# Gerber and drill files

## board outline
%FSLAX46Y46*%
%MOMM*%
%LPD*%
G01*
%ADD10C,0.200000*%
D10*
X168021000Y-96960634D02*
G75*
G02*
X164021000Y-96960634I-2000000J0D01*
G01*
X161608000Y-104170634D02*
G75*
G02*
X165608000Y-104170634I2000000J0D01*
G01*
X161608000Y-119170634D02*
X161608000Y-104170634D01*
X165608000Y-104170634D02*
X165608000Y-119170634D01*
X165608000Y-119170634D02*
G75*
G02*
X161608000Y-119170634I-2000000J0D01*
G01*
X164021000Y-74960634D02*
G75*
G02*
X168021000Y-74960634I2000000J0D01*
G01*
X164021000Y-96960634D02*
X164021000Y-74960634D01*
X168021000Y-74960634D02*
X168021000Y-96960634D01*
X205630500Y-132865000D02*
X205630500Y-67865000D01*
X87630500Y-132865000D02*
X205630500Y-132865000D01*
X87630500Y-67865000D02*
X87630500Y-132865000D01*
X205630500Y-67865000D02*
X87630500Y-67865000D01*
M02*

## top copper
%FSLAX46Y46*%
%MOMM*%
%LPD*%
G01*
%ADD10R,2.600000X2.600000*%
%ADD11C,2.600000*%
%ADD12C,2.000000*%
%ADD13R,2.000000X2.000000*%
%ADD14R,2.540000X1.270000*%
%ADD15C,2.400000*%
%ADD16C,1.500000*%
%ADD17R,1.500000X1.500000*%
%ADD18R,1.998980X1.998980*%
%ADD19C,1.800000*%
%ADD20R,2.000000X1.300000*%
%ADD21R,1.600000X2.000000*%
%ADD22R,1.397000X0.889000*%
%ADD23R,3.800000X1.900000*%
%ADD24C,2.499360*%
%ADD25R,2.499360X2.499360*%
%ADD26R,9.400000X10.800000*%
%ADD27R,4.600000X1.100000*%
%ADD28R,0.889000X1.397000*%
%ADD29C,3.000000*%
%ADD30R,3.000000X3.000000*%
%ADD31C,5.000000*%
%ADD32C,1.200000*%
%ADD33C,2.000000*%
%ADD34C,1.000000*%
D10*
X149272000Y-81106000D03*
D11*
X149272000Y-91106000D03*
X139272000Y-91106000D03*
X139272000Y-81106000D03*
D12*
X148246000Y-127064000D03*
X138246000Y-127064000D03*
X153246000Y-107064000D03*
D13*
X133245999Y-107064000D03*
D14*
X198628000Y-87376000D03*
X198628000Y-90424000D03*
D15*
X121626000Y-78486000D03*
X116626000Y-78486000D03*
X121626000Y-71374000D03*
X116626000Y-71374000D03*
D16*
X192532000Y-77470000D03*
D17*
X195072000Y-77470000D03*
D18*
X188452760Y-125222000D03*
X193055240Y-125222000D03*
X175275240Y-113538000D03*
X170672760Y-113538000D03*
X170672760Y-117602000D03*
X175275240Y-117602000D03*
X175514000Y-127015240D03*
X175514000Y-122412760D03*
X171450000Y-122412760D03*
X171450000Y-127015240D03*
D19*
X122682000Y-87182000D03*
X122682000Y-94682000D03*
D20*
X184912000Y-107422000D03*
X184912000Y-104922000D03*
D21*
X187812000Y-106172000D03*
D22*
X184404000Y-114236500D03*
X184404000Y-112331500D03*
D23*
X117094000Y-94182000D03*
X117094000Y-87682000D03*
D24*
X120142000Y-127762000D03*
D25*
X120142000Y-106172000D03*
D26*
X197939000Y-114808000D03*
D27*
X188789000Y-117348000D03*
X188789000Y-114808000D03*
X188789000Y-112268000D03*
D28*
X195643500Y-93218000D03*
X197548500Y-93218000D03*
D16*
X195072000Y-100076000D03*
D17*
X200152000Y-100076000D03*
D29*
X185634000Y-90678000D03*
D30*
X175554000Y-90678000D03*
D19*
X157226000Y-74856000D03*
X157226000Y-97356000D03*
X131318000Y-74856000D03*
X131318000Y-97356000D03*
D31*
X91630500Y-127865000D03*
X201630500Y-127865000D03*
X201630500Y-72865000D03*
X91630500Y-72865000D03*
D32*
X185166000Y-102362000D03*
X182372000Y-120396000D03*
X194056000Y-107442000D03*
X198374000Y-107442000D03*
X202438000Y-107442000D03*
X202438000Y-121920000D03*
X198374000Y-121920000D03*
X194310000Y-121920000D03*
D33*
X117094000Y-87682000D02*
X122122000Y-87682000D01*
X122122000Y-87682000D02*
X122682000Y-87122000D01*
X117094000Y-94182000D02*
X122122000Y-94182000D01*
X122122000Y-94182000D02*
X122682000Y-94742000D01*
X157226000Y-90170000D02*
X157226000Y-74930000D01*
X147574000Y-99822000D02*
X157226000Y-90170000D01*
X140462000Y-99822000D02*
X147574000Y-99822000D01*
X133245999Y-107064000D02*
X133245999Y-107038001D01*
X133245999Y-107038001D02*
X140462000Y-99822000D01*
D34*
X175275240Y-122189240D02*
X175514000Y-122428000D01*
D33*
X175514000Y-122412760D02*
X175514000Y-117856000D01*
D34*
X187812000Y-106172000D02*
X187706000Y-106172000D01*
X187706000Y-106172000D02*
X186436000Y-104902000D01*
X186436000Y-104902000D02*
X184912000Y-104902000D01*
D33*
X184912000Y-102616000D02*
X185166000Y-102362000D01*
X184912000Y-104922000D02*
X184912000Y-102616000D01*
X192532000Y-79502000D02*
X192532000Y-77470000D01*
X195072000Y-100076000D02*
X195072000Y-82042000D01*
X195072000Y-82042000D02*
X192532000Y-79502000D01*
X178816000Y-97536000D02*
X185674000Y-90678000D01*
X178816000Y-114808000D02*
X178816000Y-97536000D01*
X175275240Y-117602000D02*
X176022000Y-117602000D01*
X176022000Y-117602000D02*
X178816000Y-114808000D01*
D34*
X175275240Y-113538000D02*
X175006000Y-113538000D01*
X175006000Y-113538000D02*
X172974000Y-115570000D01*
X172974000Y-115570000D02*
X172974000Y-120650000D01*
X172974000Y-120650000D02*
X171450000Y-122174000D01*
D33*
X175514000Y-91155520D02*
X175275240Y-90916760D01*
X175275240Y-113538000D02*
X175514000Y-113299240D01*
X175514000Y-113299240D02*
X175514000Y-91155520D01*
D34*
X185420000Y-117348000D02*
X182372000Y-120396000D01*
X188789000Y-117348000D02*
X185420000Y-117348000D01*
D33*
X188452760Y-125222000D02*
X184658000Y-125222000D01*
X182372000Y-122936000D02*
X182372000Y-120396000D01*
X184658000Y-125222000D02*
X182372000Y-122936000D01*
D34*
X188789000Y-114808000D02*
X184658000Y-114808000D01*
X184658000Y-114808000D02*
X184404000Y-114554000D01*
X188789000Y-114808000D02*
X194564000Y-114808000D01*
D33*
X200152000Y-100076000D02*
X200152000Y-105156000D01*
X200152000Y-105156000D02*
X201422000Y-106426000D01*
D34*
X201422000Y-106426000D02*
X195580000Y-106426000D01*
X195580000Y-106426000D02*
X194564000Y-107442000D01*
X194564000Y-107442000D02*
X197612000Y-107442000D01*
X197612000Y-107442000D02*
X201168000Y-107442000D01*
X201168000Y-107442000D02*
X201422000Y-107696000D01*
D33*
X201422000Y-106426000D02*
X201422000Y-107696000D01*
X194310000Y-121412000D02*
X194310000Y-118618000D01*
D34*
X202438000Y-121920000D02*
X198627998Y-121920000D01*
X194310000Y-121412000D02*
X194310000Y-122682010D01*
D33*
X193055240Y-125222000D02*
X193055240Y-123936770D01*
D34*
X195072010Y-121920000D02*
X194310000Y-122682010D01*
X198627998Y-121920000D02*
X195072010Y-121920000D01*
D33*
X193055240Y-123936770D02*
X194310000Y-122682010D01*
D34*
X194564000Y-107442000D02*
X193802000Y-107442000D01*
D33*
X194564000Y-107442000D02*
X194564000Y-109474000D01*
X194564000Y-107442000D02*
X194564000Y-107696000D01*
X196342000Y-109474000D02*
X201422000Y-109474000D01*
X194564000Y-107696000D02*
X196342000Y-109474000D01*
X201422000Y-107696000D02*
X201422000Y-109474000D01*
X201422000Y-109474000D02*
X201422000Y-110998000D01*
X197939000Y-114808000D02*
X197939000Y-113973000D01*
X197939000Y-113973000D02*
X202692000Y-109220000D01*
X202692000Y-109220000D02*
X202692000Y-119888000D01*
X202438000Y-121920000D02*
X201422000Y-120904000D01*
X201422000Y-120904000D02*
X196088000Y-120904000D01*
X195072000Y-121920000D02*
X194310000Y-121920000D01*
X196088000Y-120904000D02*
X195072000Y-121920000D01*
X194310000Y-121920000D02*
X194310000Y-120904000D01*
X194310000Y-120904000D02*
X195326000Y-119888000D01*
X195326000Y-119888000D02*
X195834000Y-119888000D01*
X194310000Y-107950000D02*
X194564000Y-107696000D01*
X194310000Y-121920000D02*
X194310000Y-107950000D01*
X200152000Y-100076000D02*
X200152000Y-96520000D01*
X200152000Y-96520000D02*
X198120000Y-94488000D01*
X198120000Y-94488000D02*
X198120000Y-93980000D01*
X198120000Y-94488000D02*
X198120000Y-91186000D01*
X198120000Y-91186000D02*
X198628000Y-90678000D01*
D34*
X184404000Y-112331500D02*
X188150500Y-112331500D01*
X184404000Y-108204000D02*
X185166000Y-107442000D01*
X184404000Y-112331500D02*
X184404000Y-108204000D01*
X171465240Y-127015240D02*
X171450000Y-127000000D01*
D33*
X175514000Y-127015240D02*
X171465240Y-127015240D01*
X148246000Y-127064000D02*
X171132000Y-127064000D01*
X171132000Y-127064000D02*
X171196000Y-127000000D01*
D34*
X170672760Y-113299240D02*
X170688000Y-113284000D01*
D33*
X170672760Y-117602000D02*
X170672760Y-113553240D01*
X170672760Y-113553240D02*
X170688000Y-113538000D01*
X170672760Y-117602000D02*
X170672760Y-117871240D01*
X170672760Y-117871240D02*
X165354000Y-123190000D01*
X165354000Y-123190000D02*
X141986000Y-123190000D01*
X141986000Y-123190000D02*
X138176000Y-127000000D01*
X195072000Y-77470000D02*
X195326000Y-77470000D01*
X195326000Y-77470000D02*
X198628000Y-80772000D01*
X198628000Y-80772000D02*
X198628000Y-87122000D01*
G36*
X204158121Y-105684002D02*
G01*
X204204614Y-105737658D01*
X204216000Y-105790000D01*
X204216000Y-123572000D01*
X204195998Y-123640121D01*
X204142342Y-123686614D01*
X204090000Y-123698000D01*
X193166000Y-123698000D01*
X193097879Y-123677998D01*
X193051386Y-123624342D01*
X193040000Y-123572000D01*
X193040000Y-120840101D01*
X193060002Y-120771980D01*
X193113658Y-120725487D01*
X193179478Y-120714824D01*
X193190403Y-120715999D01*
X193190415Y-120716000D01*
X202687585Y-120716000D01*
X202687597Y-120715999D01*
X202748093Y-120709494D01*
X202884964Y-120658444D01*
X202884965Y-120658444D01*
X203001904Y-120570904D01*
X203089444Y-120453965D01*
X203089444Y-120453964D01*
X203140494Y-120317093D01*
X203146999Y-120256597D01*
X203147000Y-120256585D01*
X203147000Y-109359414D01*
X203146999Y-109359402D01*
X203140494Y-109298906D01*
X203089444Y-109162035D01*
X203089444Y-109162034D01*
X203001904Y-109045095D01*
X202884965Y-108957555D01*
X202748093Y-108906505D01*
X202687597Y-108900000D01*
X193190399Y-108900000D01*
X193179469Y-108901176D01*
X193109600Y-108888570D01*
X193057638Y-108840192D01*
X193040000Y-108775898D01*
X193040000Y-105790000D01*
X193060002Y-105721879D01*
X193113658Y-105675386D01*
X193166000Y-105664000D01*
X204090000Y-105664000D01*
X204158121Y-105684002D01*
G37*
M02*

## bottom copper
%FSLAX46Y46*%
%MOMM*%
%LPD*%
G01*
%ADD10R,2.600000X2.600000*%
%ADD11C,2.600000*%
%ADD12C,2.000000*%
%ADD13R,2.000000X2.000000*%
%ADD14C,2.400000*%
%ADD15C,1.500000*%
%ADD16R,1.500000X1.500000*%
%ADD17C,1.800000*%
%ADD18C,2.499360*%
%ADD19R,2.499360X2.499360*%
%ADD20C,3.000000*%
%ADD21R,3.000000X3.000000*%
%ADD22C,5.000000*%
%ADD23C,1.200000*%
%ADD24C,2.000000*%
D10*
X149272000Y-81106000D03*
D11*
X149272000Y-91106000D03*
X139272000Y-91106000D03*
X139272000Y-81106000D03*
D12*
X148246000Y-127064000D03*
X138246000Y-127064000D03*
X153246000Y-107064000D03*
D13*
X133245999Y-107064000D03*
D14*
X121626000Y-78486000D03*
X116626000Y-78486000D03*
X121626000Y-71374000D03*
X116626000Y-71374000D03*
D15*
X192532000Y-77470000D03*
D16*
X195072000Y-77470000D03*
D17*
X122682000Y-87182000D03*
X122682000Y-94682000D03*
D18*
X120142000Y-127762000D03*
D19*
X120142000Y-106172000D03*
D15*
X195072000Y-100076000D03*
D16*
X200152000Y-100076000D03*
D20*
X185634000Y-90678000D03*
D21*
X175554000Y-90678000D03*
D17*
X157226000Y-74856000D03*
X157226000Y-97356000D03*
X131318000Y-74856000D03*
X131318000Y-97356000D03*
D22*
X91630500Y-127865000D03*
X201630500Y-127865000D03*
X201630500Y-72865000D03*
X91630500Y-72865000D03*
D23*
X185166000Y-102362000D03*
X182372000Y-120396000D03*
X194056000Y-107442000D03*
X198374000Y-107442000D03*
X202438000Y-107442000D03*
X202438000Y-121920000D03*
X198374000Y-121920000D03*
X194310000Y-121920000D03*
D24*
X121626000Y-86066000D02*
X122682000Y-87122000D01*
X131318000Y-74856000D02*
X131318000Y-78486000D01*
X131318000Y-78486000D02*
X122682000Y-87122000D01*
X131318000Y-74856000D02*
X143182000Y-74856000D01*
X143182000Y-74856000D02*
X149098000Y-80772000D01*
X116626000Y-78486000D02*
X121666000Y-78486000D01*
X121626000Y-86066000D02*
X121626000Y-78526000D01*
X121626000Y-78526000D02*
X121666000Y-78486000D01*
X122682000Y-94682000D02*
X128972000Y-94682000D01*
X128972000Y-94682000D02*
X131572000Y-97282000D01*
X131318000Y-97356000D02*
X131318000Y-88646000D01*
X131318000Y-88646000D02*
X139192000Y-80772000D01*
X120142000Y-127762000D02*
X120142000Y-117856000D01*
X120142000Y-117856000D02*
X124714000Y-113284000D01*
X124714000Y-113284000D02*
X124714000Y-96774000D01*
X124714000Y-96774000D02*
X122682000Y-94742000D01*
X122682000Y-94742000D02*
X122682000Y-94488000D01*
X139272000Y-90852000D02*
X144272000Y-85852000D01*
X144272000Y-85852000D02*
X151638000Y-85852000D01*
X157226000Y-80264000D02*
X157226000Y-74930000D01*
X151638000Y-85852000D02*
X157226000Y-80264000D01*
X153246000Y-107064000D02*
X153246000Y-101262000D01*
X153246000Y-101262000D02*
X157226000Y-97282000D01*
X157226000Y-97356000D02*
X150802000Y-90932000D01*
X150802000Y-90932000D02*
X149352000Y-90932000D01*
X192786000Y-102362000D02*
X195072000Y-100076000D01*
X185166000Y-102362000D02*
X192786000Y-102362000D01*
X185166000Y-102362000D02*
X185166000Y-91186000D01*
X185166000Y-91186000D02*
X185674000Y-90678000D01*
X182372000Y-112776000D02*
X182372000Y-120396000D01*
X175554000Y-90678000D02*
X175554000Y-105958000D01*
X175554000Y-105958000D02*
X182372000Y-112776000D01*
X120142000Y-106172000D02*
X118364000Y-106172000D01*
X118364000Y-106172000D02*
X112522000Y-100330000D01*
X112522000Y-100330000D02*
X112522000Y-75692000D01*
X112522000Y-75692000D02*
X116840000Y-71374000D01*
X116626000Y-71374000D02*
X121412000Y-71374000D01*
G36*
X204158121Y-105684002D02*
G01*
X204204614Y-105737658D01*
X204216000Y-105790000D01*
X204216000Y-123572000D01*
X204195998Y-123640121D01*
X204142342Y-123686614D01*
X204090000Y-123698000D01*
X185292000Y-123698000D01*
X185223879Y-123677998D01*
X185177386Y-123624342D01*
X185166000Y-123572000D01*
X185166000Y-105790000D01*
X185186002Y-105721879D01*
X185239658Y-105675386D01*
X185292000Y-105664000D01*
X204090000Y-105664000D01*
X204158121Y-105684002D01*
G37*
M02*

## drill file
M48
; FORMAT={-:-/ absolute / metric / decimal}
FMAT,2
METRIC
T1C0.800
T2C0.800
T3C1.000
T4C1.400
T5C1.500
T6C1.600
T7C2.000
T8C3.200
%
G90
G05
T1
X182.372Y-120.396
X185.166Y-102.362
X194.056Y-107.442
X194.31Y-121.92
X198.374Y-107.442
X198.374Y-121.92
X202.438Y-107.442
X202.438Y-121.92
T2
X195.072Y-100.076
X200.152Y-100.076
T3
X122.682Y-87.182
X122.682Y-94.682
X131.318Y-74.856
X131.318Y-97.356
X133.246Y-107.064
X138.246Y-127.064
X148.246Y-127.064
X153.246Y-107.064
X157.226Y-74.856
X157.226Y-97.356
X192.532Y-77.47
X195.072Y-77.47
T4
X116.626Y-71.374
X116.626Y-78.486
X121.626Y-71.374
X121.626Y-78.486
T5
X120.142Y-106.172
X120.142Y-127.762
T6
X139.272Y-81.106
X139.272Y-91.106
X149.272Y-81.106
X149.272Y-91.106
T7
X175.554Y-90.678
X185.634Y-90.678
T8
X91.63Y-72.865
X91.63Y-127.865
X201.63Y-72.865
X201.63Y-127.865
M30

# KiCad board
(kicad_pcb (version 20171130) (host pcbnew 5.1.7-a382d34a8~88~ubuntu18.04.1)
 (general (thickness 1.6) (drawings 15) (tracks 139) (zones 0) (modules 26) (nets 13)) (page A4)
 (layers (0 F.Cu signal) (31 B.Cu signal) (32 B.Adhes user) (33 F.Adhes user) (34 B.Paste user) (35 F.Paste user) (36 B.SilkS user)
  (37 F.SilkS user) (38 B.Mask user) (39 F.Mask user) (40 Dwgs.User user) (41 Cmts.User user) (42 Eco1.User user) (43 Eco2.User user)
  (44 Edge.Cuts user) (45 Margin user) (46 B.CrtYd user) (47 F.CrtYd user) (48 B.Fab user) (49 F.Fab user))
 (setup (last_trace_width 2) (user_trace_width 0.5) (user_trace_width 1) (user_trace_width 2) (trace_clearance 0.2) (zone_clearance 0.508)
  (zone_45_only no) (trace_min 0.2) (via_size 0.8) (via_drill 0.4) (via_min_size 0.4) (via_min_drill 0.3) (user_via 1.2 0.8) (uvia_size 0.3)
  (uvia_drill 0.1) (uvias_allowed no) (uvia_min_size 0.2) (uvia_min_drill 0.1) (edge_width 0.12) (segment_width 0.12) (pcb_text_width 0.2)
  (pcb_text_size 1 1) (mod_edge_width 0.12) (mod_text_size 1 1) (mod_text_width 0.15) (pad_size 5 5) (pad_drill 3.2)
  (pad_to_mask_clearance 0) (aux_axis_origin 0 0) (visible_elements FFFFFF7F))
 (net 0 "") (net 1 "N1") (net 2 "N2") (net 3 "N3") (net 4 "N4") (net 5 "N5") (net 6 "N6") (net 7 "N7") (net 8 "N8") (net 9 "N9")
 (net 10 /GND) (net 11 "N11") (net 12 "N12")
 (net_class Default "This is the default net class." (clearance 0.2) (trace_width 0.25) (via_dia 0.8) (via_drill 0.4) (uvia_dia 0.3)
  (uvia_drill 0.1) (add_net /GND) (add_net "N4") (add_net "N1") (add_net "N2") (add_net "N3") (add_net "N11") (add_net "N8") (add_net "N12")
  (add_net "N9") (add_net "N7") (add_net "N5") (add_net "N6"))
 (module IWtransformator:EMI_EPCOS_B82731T (layer F.Cu) (at 144.272 86.106 270)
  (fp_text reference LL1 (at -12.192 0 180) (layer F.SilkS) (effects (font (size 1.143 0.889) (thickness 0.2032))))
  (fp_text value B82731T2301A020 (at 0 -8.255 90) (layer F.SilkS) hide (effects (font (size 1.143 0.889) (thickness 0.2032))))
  (pad 1 thru_hole rect (at -5 -5 270) (size 2.6 2.6) (drill 1.6) (layers *.Cu *.Mask) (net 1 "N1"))
  (pad 4 thru_hole circle (at 5 -5 270) (size 2.6 2.6) (drill 1.6) (layers *.Cu *.Mask) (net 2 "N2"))
  (pad 3 thru_hole circle (at 5 5 270) (size 2.6 2.6) (drill 1.6) (layers *.Cu *.Mask) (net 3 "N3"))
  (pad 2 thru_hole circle (at -5 5 270) (size 2.6 2.6) (drill 1.6) (layers *.Cu *.Mask) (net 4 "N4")))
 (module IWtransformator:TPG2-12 (layer F.Cu) (at 143.256 117.094)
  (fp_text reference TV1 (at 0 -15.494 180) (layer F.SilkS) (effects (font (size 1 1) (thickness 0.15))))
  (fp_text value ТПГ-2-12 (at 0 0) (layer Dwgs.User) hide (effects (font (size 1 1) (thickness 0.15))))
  (pad 7 thru_hole circle (at 4.99 9.97) (size 2 2) (drill 1) (layers *.Cu *.Mask) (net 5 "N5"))
  (pad 9 thru_hole circle (at -5.01 9.97) (size 2 2) (drill 1) (layers *.Cu *.Mask) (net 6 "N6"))
  (pad 5 thru_hole circle (at 9.99 -10.03) (size 2 2) (drill 1) (layers *.Cu *.Mask) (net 2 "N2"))
  (pad 1 thru_hole rect (at -10.010001 -10.03) (size 2 2) (drill 1) (layers *.Cu *.Mask) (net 3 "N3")))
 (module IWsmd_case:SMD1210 (layer F.Cu) (at 198.628 88.9 90)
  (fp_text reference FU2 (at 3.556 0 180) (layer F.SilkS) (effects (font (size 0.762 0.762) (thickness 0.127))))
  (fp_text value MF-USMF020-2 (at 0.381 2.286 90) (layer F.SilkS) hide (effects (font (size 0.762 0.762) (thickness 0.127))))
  (pad 2 smd rect (at 1.524 0 90) (size 1.27 2.54) (layers F.Cu F.Paste F.Mask) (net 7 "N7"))
  (pad 1 smd rect (at -1.524 0 90) (size 1.27 2.54) (layers F.Cu F.Paste F.Mask) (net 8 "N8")))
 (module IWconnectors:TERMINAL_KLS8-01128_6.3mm (layer F.Cu) (at 119.126 78.486)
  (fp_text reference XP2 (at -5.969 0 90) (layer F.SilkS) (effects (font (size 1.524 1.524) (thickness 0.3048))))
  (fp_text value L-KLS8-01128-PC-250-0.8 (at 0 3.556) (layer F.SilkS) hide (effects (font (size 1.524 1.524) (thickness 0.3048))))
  (pad 1 thru_hole circle (at 2.5 0) (size 2.4 2.4) (drill 1.4) (layers *.Cu *.Mask) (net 1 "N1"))
  (pad 1 thru_hole circle (at -2.5 0) (size 2.4 2.4) (drill 1.4) (layers *.Cu *.Mask) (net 1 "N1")))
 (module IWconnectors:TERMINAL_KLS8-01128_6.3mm (layer F.Cu) (at 119.126 71.374)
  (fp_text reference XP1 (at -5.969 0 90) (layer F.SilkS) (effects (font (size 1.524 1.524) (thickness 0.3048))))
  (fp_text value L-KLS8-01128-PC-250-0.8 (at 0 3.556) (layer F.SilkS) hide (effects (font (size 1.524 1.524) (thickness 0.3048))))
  (pad 1 thru_hole circle (at 2.5 0) (size 2.4 2.4) (drill 1.4) (layers *.Cu *.Mask) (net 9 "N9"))
  (pad 1 thru_hole circle (at -2.5 0) (size 2.4 2.4) (drill 1.4) (layers *.Cu *.Mask) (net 9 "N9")))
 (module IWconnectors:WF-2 (layer F.Cu) (at 193.802 77.47 180)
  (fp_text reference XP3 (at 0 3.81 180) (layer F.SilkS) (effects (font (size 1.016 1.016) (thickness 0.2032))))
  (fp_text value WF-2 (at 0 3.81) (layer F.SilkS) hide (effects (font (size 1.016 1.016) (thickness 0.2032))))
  (pad 2 thru_hole circle (at 1.27 0 180) (size 1.5 1.5) (drill 1) (layers *.Cu *.Mask) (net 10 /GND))
  (pad 1 thru_hole rect (at -1.27 0 180) (size 1.5 1.5) (drill 1) (layers *.Cu *.Mask) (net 7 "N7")))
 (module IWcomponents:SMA (layer F.Cu) (at 190.754 125.222 180)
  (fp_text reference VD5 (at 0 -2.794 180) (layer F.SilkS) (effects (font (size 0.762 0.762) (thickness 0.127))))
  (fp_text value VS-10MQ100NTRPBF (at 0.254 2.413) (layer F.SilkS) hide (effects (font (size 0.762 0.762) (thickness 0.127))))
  (pad 2 smd rect (at 2.30124 0 180) (size 1.99898 1.99898) (layers F.Cu F.Paste F.Mask) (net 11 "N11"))
  (pad 1 smd rect (at -2.30124 0 180) (size 1.99898 1.99898) (layers F.Cu F.Paste F.Mask) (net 8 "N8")))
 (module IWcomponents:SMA (layer F.Cu) (at 172.974 113.538)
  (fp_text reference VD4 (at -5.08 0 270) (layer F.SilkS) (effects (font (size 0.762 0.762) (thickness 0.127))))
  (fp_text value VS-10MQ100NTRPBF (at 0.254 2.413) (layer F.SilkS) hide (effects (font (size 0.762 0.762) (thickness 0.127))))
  (pad 2 smd rect (at 2.30124 0) (size 1.99898 1.99898) (layers F.Cu F.Paste F.Mask) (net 11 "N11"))
  (pad 1 smd rect (at -2.30124 0) (size 1.99898 1.99898) (layers F.Cu F.Paste F.Mask) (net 6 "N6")))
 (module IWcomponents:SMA (layer F.Cu) (at 172.974 117.602 180)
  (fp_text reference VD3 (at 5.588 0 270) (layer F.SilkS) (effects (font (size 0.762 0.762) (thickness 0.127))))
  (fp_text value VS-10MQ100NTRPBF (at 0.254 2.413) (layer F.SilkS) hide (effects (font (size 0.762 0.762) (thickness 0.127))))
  (pad 2 smd rect (at 2.30124 0 180) (size 1.99898 1.99898) (layers F.Cu F.Paste F.Mask) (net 6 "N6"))
  (pad 1 smd rect (at -2.30124 0 180) (size 1.99898 1.99898) (layers F.Cu F.Paste F.Mask) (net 10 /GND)))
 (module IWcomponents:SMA (layer F.Cu) (at 175.514 124.714 270)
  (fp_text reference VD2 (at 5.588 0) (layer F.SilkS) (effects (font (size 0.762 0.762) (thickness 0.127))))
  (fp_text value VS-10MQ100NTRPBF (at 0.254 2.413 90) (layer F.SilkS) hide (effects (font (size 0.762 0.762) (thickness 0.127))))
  (pad 2 smd rect (at 2.30124 0 270) (size 1.99898 1.99898) (layers F.Cu F.Paste F.Mask) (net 5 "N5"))
  (pad 1 smd rect (at -2.30124 0 270) (size 1.99898 1.99898) (layers F.Cu F.Paste F.Mask) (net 10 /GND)))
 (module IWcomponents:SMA (layer F.Cu) (at 171.45 124.714 90)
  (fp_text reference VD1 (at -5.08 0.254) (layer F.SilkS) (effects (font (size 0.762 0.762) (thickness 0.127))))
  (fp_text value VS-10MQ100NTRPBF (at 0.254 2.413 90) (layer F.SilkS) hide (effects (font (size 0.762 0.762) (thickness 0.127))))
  (pad 2 smd rect (at 2.30124 0 90) (size 1.99898 1.99898) (layers F.Cu F.Paste F.Mask) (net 11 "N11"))
  (pad 1 smd rect (at -2.30124 0 90) (size 1.99898 1.99898) (layers F.Cu F.Paste F.Mask) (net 5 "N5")))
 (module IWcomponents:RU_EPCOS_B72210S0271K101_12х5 (layer F.Cu) (at 122.682 90.932 90)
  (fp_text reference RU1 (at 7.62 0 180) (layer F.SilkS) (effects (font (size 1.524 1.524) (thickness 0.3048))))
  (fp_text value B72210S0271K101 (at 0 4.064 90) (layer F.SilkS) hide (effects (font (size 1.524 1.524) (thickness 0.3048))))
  (pad 2 thru_hole circle (at 3.75 0 90) (size 1.8 1.8) (drill 1) (layers *.Cu *.Mask) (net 1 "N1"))
  (pad 1 thru_hole circle (at -3.75 0 90) (size 1.8 1.8) (drill 1) (layers *.Cu *.Mask) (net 4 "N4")))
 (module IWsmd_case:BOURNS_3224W (layer F.Cu) (at 184.912 106.172 90)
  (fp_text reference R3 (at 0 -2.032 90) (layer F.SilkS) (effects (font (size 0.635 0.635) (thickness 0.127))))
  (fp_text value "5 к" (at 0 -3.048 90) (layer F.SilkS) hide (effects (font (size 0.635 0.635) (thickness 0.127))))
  (pad 1 smd rect (at -1.25 0 90) (size 1.3 2) (layers F.Cu F.Paste F.Mask) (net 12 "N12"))
  (pad 3 smd rect (at 1.25 0 90) (size 1.3 2) (layers F.Cu F.Paste F.Mask) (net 10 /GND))
  (pad 2 smd rect (at 0 2.9 90) (size 2 1.6) (layers F.Cu F.Paste F.Mask) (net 10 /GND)))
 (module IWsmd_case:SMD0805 (layer F.Cu) (at 184.404 113.284 270)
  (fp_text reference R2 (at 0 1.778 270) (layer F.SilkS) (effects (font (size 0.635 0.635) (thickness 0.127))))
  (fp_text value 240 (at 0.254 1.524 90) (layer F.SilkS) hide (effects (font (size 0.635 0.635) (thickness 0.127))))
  (pad 2 smd rect (at 0.9525 0 270) (size 0.889 1.397) (layers F.Cu F.Paste F.Mask) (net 8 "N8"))
  (pad 1 smd rect (at -0.9525 0 270) (size 0.889 1.397) (layers F.Cu F.Paste F.Mask) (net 12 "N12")))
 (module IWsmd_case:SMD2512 (layer F.Cu) (at 117.094 90.932 270)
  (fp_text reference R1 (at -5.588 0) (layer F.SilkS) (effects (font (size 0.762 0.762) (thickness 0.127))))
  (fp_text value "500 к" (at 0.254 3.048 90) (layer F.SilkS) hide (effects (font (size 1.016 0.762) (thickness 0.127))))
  (pad 2 smd rect (at 3.25 0 270) (size 1.9 3.8) (layers F.Cu F.Paste F.Mask) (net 4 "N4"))
  (pad 1 smd rect (at -3.25 0 270) (size 1.9 3.8) (layers F.Cu F.Paste F.Mask) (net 1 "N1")))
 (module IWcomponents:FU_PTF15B (layer F.Cu) (at 120.142 111.252 270)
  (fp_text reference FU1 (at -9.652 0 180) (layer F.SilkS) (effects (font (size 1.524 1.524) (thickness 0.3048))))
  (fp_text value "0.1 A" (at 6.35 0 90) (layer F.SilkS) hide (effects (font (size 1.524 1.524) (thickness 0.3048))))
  (pad 2 thru_hole circle (at 16.51 0 270) (size 2.49936 2.49936) (drill 1.5) (layers *.Cu *.Mask) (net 4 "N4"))
  (pad 1 thru_hole rect (at -5.08 0 270) (size 2.49936 2.49936) (drill 1.5) (layers *.Cu *.Mask) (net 9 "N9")))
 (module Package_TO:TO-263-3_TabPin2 (layer F.Cu) (at 194.564 114.808)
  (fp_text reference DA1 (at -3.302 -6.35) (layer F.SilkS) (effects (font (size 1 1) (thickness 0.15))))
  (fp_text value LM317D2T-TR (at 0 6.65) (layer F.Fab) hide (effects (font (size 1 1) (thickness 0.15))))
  (pad "" smd rect (at 0.95 2.775) (size 4.55 5.25) (layers F.Paste))
  (pad "" smd rect (at 5.8 -2.775) (size 4.55 5.25) (layers F.Paste))
  (pad "" smd rect (at 0.95 -2.775) (size 4.55 5.25) (layers F.Paste))
  (pad "" smd rect (at 5.8 2.775) (size 4.55 5.25) (layers F.Paste))
  (pad 2 smd rect (at 3.375 0) (size 9.4 10.8) (layers F.Cu F.Mask) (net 8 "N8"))
  (pad 3 smd rect (at -5.775 2.54) (size 4.6 1.1) (layers F.Cu F.Paste F.Mask) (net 11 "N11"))
  (pad 2 smd rect (at -5.775 0) (size 4.6 1.1) (layers F.Cu F.Paste F.Mask) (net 8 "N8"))
  (pad 1 smd rect (at -5.775 -2.54) (size 4.6 1.1) (layers F.Cu F.Paste F.Mask) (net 12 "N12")))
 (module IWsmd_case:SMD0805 (layer F.Cu) (at 196.596 93.218 180)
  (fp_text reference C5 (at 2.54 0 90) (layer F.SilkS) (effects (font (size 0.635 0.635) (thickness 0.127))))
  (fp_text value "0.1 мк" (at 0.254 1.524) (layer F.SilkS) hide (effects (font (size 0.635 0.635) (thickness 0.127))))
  (pad 2 smd rect (at 0.9525 0 180) (size 0.889 1.397) (layers F.Cu F.Paste F.Mask) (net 10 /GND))
  (pad 1 smd rect (at -0.9525 0 180) (size 0.889 1.397) (layers F.Cu F.Paste F.Mask) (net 8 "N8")))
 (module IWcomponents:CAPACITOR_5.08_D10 (layer F.Cu) (at 197.612 100.076 180)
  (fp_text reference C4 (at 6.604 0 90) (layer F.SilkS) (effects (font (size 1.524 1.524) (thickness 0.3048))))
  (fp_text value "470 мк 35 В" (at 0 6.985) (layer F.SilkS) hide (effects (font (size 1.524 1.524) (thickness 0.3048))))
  (pad 2 thru_hole circle (at 2.54 0 180) (size 1.5 1.5) (drill 0.8) (layers *.Cu *.Mask) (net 10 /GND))
  (pad 1 thru_hole rect (at -2.54 0 180) (size 1.5 1.5) (drill 0.8) (layers *.Cu *.Mask) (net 8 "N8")))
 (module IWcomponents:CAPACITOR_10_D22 (layer F.Cu) (at 180.594 90.678)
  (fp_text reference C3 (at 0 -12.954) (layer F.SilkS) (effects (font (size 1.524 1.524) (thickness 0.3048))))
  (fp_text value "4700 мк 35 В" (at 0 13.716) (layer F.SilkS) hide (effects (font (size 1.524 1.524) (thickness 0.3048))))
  (pad 2 thru_hole circle (at 5.04 0) (size 3 3) (drill 2) (layers *.Cu *.Mask) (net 10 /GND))
  (pad 1 thru_hole rect (at -5.04 0) (size 3 3) (drill 2) (layers *.Cu *.Mask) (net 11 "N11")))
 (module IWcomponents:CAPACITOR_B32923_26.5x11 (layer F.Cu) (at 157.226 86.106 90)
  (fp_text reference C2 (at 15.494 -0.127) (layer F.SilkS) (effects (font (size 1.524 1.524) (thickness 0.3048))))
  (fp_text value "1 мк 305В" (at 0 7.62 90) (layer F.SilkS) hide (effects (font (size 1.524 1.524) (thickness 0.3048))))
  (pad 2 thru_hole circle (at 11.25 0 90) (size 1.8 1.8) (drill 1) (layers *.Cu *.Mask) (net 3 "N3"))
  (pad 1 thru_hole circle (at -11.25 0 90) (size 1.8 1.8) (drill 1) (layers *.Cu *.Mask) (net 2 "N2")))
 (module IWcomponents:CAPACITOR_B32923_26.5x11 (layer F.Cu) (at 131.318 86.106 90)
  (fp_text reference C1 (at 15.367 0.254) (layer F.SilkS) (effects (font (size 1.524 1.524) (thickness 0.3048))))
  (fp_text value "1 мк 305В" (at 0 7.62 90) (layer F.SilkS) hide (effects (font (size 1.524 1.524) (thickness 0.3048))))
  (pad 2 thru_hole circle (at 11.25 0 90) (size 1.8 1.8) (drill 1) (layers *.Cu *.Mask) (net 1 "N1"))
  (pad 1 thru_hole circle (at -11.25 0 90) (size 1.8 1.8) (drill 1) (layers *.Cu *.Mask) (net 4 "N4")))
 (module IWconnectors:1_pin (layer F.Cu) (at 91.6305 127.865)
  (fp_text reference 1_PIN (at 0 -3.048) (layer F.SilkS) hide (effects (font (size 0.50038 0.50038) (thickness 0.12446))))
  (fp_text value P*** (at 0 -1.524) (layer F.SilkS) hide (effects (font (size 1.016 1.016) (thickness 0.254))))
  (pad 1 thru_hole circle (at 0 0) (size 5 5) (drill 3.2) (layers *.Cu *.Mask)))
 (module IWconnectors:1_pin (layer F.Cu) (at 201.6305 127.865)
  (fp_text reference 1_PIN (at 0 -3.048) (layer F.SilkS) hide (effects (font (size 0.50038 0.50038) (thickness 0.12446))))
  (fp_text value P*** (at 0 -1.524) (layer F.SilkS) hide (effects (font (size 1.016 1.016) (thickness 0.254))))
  (pad 1 thru_hole circle (at 0 0) (size 5 5) (drill 3.2) (layers *.Cu *.Mask)))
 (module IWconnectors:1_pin (layer F.Cu) (at 201.6305 72.865)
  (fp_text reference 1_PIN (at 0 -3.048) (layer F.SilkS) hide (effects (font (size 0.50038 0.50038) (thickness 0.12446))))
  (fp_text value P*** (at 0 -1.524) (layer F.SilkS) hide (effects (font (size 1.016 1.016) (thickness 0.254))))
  (pad 1 thru_hole circle (at 0 0) (size 5 5) (drill 3.2) (layers *.Cu *.Mask)))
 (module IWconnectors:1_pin (layer F.Cu) (at 91.6305 72.865)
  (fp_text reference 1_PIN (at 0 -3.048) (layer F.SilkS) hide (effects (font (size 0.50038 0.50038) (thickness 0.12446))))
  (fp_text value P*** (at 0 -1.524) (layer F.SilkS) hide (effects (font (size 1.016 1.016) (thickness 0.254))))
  (pad 1 thru_hole circle (at 0 0) (size 5 5) (drill 3.2) (layers *.Cu *.Mask)))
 (gr_arc (start 166.021 96.960634) (end 164.021 96.960634) (angle -180) (layer Edge.Cuts) (width 0.2))
 (gr_arc (start 163.608 104.170634) (end 165.608 104.170634) (angle -180) (layer Edge.Cuts) (width 0.2))
 (gr_line (start 161.608 119.170634) (end 161.608 104.170634) (layer Edge.Cuts) (width 0.2))
 (gr_line (start 165.608 104.170634) (end 165.608 119.170634) (layer Edge.Cuts) (width 0.2))
 (gr_arc (start 163.608 119.170634) (end 161.608 119.170634) (angle -180) (layer Edge.Cuts) (width 0.2))
 (gr_arc (start 166.021 74.960634) (end 168.021 74.960634) (angle -180) (layer Edge.Cuts) (width 0.2))
 (gr_line (start 164.021 96.960634) (end 164.021 74.960634) (layer Edge.Cuts) (width 0.2))
 (gr_line (start 168.021 74.960634) (end 168.021 96.960634) (layer Edge.Cuts) (width 0.2))
 (gr_line (start 205.6305 132.865) (end 205.6305 67.865) (layer Edge.Cuts) (width 0.2))
 (gr_line (start 87.6305 132.865) (end 205.6305 132.865) (layer Edge.Cuts) (width 0.2))
 (gr_line (start 87.6305 67.865) (end 87.6305 132.865) (layer Edge.Cuts) (width 0.2))
 (gr_line (start 205.6305 67.865) (end 87.6305 67.865) (layer Edge.Cuts) (width 0.2))
 (segment (start 121.626 86.066) (end 122.682 87.122) (width 2) (layer B.Cu) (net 1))
 (segment (start 117.094 87.682) (end 122.122 87.682) (width 2) (layer F.Cu) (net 1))
 (segment (start 122.122 87.682) (end 122.682 87.122) (width 2) (layer F.Cu) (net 1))
 (segment (start 131.318 74.856) (end 131.318 78.486) (width 2) (layer B.Cu) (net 1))
 (segment (start 131.318 78.486) (end 122.682 87.122) (width 2) (layer B.Cu) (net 1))
 (segment (start 131.318 74.856) (end 143.182 74.856) (width 2) (layer B.Cu) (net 1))
 (segment (start 143.182 74.856) (end 149.098 80.772) (width 2) (layer B.Cu) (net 1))
 (segment (start 116.626 78.486) (end 121.666 78.486) (width 2) (layer B.Cu) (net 1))
 (segment (start 121.626 86.066) (end 121.626 78.526) (width 2) (layer B.Cu) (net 1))
 (segment (start 121.626 78.526) (end 121.666 78.486) (width 2) (layer B.Cu) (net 1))
 (segment (start 117.094 94.182) (end 122.122 94.182) (width 2) (layer F.Cu) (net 4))
 (segment (start 122.122 94.182) (end 122.682 94.742) (width 2) (layer F.Cu) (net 4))
 (segment (start 122.682 94.682) (end 128.972 94.682) (width 2) (layer B.Cu) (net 4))
 (segment (start 128.972 94.682) (end 131.572 97.282) (width 2) (layer B.Cu) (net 4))
 (segment (start 131.318 97.356) (end 131.318 88.646) (width 2) (layer B.Cu) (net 4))
 (segment (start 131.318 88.646) (end 139.192 80.772) (width 2) (layer B.Cu) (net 4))
 (segment (start 120.142 127.762) (end 120.142 117.856) (width 2) (layer B.Cu) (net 4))
 (segment (start 120.142 117.856) (end 124.714 113.284) (width 2) (layer B.Cu) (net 4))
 (segment (start 124.714 113.284) (end 124.714 96.774) (width 2) (layer B.Cu) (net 4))
 (segment (start 124.714 96.774) (end 122.682 94.742) (width 2) (layer B.Cu) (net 4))
 (segment (start 122.682 94.742) (end 122.682 94.488) (width 2) (layer B.Cu) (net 4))
 (segment (start 139.272 90.852) (end 144.272 85.852) (width 2) (layer B.Cu) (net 3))
 (segment (start 144.272 85.852) (end 151.638 85.852) (width 2) (layer B.Cu) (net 3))
 (segment (start 157.226 80.264) (end 157.226 74.93) (width 2) (layer B.Cu) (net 3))
 (segment (start 151.638 85.852) (end 157.226 80.264) (width 2) (layer B.Cu) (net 3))
 (segment (start 157.226 90.17) (end 157.226 74.93) (width 2) (layer F.Cu) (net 3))
 (segment (start 147.574 99.822) (end 157.226 90.17) (width 2) (layer F.Cu) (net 3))
 (segment (start 140.462 99.822) (end 147.574 99.822) (width 2) (layer F.Cu) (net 3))
 (segment (start 133.245999 107.064) (end 133.245999 107.038001) (width 2) (layer F.Cu) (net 3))
 (segment (start 133.245999 107.038001) (end 140.462 99.822) (width 2) (layer F.Cu) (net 3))
 (segment (start 153.246 107.064) (end 153.246 101.262) (width 2) (layer B.Cu) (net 2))
 (segment (start 153.246 101.262) (end 157.226 97.282) (width 2) (layer B.Cu) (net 2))
 (segment (start 157.226 97.356) (end 150.802 90.932) (width 2) (layer B.Cu) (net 2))
 (segment (start 150.802 90.932) (end 149.352 90.932) (width 2) (layer B.Cu) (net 2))
 (segment (start 175.27524 122.18924) (end 175.514 122.428) (width 1) (layer F.Cu) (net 10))
 (segment (start 175.514 122.41276) (end 175.514 117.856) (width 2) (layer F.Cu) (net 10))
 (segment (start 187.812 106.172) (end 187.706 106.172) (width 1) (layer F.Cu) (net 10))
 (segment (start 187.706 106.172) (end 186.436 104.902) (width 1) (layer F.Cu) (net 10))
 (segment (start 186.436 104.902) (end 184.912 104.902) (width 1) (layer F.Cu) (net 10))
 (segment (start 192.786 102.362) (end 195.072 100.076) (width 2) (layer B.Cu) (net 10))
 (via (at 185.166 102.362) (size 1.2) (drill 0.8) (layers F.Cu B.Cu) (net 10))
 (segment (start 185.166 102.362) (end 192.786 102.362) (width 2) (layer B.Cu) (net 10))
 (segment (start 185.166 102.362) (end 185.166 91.186) (width 2) (layer B.Cu) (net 10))
 (segment (start 185.166 91.186) (end 185.674 90.678) (width 2) (layer B.Cu) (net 10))
 (segment (start 184.912 102.616) (end 185.166 102.362) (width 2) (layer F.Cu) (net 10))
 (segment (start 184.912 104.922) (end 184.912 102.616) (width 2) (layer F.Cu) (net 10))
 (segment (start 192.532 79.502) (end 192.532 77.47) (width 2) (layer F.Cu) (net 10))
 (segment (start 195.072 100.076) (end 195.072 82.042) (width 2) (layer F.Cu) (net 10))
 (segment (start 195.072 82.042) (end 192.532 79.502) (width 2) (layer F.Cu) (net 10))
 (segment (start 178.816 97.536) (end 185.674 90.678) (width 2) (layer F.Cu) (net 10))
 (segment (start 178.816 114.808) (end 178.816 97.536) (width 2) (layer F.Cu) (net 10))
 (segment (start 175.27524 117.602) (end 176.022 117.602) (width 2) (layer F.Cu) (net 10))
 (segment (start 176.022 117.602) (end 178.816 114.808) (width 2) (layer F.Cu) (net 10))
 (segment (start 175.27524 113.538) (end 175.006 113.538) (width 1) (layer F.Cu) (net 11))
 (segment (start 175.006 113.538) (end 172.974 115.57) (width 1) (layer F.Cu) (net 11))
 (segment (start 172.974 115.57) (end 172.974 120.65) (width 1) (layer F.Cu) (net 11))
 (segment (start 172.974 120.65) (end 171.45 122.174) (width 1) (layer F.Cu) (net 11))
 (segment (start 175.514 91.15552) (end 175.27524 90.91676) (width 2) (layer F.Cu) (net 11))
 (segment (start 175.27524 113.538) (end 175.514 113.29924) (width 2) (layer F.Cu) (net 11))
 (segment (start 175.514 113.29924) (end 175.514 91.15552) (width 2) (layer F.Cu) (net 11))
 (via (at 182.372 120.396) (size 1.2) (drill 0.8) (layers F.Cu B.Cu) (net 11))
 (segment (start 185.42 117.348) (end 182.372 120.396) (width 1) (layer F.Cu) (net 11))
 (segment (start 188.789 117.348) (end 185.42 117.348) (width 1) (layer F.Cu) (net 11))
 (segment (start 188.45276 125.222) (end 184.658 125.222) (width 2) (layer F.Cu) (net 11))
 (segment (start 182.372 122.936) (end 182.372 120.396) (width 2) (layer F.Cu) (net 11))
 (segment (start 184.658 125.222) (end 182.372 122.936) (width 2) (layer F.Cu) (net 11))
 (segment (start 182.372 112.776) (end 182.372 120.396) (width 2) (layer B.Cu) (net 11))
 (segment (start 175.554 90.678) (end 175.554 105.958) (width 2) (layer B.Cu) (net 11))
 (segment (start 175.554 105.958) (end 182.372 112.776) (width 2) (layer B.Cu) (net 11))
 (segment (start 188.789 114.808) (end 184.658 114.808) (width 1) (layer F.Cu) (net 8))
 (segment (start 184.658 114.808) (end 184.404 114.554) (width 1) (layer F.Cu) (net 8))
 (segment (start 188.789 114.808) (end 194.564 114.808) (width 1) (layer F.Cu) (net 8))
 (segment (start 200.152 100.076) (end 200.152 105.156) (width 2) (layer F.Cu) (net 8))
 (segment (start 200.152 105.156) (end 201.422 106.426) (width 2) (layer F.Cu) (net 8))
 (via (at 194.056 107.442) (size 1.2) (drill 0.8) (layers F.Cu B.Cu) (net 8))
 (segment (start 201.422 106.426) (end 195.58 106.426) (width 1) (layer F.Cu) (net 8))
 (segment (start 195.58 106.426) (end 194.564 107.442) (width 1) (layer F.Cu) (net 8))
 (via (at 198.374 107.442) (size 1.2) (drill 0.8) (layers F.Cu B.Cu) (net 8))
 (segment (start 194.564 107.442) (end 197.612 107.442) (width 1) (layer F.Cu) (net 8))
 (via (at 202.438 107.442) (size 1.2) (drill 0.8) (layers F.Cu B.Cu) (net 8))
 (segment (start 197.612 107.442) (end 201.168 107.442) (width 1) (layer F.Cu) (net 8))
 (segment (start 201.168 107.442) (end 201.422 107.696) (width 1) (layer F.Cu) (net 8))
 (segment (start 201.422 106.426) (end 201.422 107.696) (width 2) (layer F.Cu) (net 8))
 (segment (start 194.31 121.412) (end 194.31 118.618) (width 2) (layer F.Cu) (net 8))
 (via (at 202.438 121.92) (size 1.2) (drill 0.8) (layers F.Cu B.Cu) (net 8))
 (via (at 198.374 121.92) (size 1.2) (drill 0.8) (layers F.Cu B.Cu) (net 8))
 (segment (start 202.438 121.92) (end 198.627998 121.92) (width 1) (layer F.Cu) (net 8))
 (via (at 194.31 121.92) (size 1.2) (drill 0.8) (layers F.Cu B.Cu) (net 8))
 (segment (start 194.31 121.412) (end 194.31 122.68201) (width 1) (layer F.Cu) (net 8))
 (segment (start 193.05524 125.222) (end 193.05524 123.93677) (width 2) (layer F.Cu) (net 8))
 (segment (start 195.07201 121.92) (end 194.31 122.68201) (width 1) (layer F.Cu) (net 8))
 (segment (start 198.627998 121.92) (end 195.07201 121.92) (width 1) (layer F.Cu) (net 8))
 (segment (start 193.05524 123.93677) (end 194.31 122.68201) (width 2) (layer F.Cu) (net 8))
 (segment (start 194.564 107.442) (end 193.802 107.442) (width 1) (layer F.Cu) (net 8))
 (segment (start 194.564 107.442) (end 194.564 109.474) (width 2) (layer F.Cu) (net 8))
 (segment (start 194.564 107.442) (end 194.564 107.696) (width 2) (layer F.Cu) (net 8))
 (segment (start 196.342 109.474) (end 201.422 109.474) (width 2) (layer F.Cu) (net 8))
 (segment (start 194.564 107.696) (end 196.342 109.474) (width 2) (layer F.Cu) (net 8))
 (segment (start 201.422 107.696) (end 201.422 109.474) (width 2) (layer F.Cu) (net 8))
 (segment (start 201.422 109.474) (end 201.422 110.998) (width 2) (layer F.Cu) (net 8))
 (segment (start 197.939 114.808) (end 197.939 113.973) (width 2) (layer F.Cu) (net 8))
 (segment (start 197.939 113.973) (end 202.692 109.22) (width 2) (layer F.Cu) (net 8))
 (segment (start 202.692 109.22) (end 202.692 119.888) (width 2) (layer F.Cu) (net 8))
 (segment (start 202.438 121.92) (end 201.422 120.904) (width 2) (layer F.Cu) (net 8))
 (segment (start 201.422 120.904) (end 196.088 120.904) (width 2) (layer F.Cu) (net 8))
 (segment (start 195.072 121.92) (end 194.31 121.92) (width 2) (layer F.Cu) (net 8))
 (segment (start 196.088 120.904) (end 195.072 121.92) (width 2) (layer F.Cu) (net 8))
 (segment (start 194.31 121.92) (end 194.31 120.904) (width 2) (layer F.Cu) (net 8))
 (segment (start 194.31 120.904) (end 195.326 119.888) (width 2) (layer F.Cu) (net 8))
 (segment (start 195.326 119.888) (end 195.834 119.888) (width 2) (layer F.Cu) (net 8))
 (segment (start 194.31 107.95) (end 194.564 107.696) (width 2) (layer F.Cu) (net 8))
 (segment (start 194.31 121.92) (end 194.31 107.95) (width 2) (layer F.Cu) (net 8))
 (segment (start 200.152 100.076) (end 200.152 96.52) (width 2) (layer F.Cu) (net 8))
 (segment (start 200.152 96.52) (end 198.12 94.488) (width 2) (layer F.Cu) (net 8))
 (segment (start 198.12 94.488) (end 198.12 93.98) (width 2) (layer F.Cu) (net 8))
 (segment (start 198.12 94.488) (end 198.12 91.186) (width 2) (layer F.Cu) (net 8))
 (segment (start 198.12 91.186) (end 198.628 90.678) (width 2) (layer F.Cu) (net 8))
 (segment (start 184.404 112.3315) (end 188.1505 112.3315) (width 1) (layer F.Cu) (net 12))
 (segment (start 184.404 108.204) (end 185.166 107.442) (width 1) (layer F.Cu) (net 12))
 (segment (start 184.404 112.3315) (end 184.404 108.204) (width 1) (layer F.Cu) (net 12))
 (segment (start 120.142 106.172) (end 118.364 106.172) (width 2) (layer B.Cu) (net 9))
 (segment (start 118.364 106.172) (end 112.522 100.33) (width 2) (layer B.Cu) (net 9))
 (segment (start 112.522 100.33) (end 112.522 75.692) (width 2) (layer B.Cu) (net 9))
 (segment (start 112.522 75.692) (end 116.84 71.374) (width 2) (layer B.Cu) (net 9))
 (segment (start 116.626 71.374) (end 121.412 71.374) (width 2) (layer B.Cu) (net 9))
 (segment (start 171.46524 127.01524) (end 171.45 127) (width 1) (layer F.Cu) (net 5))
 (segment (start 175.514 127.01524) (end 171.46524 127.01524) (width 2) (layer F.Cu) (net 5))
 (segment (start 148.246 127.064) (end 171.132 127.064) (width 2) (layer F.Cu) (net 5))
 (segment (start 171.132 127.064) (end 171.196 127) (width 2) (layer F.Cu) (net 5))
 (segment (start 170.67276 113.29924) (end 170.688 113.284) (width 1) (layer F.Cu) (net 6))
 (segment (start 170.67276 117.602) (end 170.67276 113.55324) (width 2) (layer F.Cu) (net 6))
 (segment (start 170.67276 113.55324) (end 170.688 113.538) (width 2) (layer F.Cu) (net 6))
 (segment (start 170.67276 117.602) (end 170.67276 117.87124) (width 2) (layer F.Cu) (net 6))
 (segment (start 170.67276 117.87124) (end 165.354 123.19) (width 2) (layer F.Cu) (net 6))
 (segment (start 165.354 123.19) (end 141.986 123.19) (width 2) (layer F.Cu) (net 6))
 (segment (start 141.986 123.19) (end 138.176 127) (width 2) (layer F.Cu) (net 6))
 (segment (start 195.072 77.47) (end 195.326 77.47) (width 2) (layer F.Cu) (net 7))
 (segment (start 195.326 77.47) (end 198.628 80.772) (width 2) (layer F.Cu) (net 7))
 (segment (start 198.628 80.772) (end 198.628 87.122) (width 2) (layer F.Cu) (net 7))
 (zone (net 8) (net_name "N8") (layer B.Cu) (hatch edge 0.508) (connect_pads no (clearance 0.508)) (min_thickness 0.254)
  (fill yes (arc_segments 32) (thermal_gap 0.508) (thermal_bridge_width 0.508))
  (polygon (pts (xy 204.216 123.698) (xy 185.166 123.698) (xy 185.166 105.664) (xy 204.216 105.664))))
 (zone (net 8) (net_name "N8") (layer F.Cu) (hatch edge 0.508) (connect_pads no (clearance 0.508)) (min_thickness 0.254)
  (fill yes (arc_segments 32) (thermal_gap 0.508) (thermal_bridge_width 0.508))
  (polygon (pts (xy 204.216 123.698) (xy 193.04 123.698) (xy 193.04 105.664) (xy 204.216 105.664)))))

